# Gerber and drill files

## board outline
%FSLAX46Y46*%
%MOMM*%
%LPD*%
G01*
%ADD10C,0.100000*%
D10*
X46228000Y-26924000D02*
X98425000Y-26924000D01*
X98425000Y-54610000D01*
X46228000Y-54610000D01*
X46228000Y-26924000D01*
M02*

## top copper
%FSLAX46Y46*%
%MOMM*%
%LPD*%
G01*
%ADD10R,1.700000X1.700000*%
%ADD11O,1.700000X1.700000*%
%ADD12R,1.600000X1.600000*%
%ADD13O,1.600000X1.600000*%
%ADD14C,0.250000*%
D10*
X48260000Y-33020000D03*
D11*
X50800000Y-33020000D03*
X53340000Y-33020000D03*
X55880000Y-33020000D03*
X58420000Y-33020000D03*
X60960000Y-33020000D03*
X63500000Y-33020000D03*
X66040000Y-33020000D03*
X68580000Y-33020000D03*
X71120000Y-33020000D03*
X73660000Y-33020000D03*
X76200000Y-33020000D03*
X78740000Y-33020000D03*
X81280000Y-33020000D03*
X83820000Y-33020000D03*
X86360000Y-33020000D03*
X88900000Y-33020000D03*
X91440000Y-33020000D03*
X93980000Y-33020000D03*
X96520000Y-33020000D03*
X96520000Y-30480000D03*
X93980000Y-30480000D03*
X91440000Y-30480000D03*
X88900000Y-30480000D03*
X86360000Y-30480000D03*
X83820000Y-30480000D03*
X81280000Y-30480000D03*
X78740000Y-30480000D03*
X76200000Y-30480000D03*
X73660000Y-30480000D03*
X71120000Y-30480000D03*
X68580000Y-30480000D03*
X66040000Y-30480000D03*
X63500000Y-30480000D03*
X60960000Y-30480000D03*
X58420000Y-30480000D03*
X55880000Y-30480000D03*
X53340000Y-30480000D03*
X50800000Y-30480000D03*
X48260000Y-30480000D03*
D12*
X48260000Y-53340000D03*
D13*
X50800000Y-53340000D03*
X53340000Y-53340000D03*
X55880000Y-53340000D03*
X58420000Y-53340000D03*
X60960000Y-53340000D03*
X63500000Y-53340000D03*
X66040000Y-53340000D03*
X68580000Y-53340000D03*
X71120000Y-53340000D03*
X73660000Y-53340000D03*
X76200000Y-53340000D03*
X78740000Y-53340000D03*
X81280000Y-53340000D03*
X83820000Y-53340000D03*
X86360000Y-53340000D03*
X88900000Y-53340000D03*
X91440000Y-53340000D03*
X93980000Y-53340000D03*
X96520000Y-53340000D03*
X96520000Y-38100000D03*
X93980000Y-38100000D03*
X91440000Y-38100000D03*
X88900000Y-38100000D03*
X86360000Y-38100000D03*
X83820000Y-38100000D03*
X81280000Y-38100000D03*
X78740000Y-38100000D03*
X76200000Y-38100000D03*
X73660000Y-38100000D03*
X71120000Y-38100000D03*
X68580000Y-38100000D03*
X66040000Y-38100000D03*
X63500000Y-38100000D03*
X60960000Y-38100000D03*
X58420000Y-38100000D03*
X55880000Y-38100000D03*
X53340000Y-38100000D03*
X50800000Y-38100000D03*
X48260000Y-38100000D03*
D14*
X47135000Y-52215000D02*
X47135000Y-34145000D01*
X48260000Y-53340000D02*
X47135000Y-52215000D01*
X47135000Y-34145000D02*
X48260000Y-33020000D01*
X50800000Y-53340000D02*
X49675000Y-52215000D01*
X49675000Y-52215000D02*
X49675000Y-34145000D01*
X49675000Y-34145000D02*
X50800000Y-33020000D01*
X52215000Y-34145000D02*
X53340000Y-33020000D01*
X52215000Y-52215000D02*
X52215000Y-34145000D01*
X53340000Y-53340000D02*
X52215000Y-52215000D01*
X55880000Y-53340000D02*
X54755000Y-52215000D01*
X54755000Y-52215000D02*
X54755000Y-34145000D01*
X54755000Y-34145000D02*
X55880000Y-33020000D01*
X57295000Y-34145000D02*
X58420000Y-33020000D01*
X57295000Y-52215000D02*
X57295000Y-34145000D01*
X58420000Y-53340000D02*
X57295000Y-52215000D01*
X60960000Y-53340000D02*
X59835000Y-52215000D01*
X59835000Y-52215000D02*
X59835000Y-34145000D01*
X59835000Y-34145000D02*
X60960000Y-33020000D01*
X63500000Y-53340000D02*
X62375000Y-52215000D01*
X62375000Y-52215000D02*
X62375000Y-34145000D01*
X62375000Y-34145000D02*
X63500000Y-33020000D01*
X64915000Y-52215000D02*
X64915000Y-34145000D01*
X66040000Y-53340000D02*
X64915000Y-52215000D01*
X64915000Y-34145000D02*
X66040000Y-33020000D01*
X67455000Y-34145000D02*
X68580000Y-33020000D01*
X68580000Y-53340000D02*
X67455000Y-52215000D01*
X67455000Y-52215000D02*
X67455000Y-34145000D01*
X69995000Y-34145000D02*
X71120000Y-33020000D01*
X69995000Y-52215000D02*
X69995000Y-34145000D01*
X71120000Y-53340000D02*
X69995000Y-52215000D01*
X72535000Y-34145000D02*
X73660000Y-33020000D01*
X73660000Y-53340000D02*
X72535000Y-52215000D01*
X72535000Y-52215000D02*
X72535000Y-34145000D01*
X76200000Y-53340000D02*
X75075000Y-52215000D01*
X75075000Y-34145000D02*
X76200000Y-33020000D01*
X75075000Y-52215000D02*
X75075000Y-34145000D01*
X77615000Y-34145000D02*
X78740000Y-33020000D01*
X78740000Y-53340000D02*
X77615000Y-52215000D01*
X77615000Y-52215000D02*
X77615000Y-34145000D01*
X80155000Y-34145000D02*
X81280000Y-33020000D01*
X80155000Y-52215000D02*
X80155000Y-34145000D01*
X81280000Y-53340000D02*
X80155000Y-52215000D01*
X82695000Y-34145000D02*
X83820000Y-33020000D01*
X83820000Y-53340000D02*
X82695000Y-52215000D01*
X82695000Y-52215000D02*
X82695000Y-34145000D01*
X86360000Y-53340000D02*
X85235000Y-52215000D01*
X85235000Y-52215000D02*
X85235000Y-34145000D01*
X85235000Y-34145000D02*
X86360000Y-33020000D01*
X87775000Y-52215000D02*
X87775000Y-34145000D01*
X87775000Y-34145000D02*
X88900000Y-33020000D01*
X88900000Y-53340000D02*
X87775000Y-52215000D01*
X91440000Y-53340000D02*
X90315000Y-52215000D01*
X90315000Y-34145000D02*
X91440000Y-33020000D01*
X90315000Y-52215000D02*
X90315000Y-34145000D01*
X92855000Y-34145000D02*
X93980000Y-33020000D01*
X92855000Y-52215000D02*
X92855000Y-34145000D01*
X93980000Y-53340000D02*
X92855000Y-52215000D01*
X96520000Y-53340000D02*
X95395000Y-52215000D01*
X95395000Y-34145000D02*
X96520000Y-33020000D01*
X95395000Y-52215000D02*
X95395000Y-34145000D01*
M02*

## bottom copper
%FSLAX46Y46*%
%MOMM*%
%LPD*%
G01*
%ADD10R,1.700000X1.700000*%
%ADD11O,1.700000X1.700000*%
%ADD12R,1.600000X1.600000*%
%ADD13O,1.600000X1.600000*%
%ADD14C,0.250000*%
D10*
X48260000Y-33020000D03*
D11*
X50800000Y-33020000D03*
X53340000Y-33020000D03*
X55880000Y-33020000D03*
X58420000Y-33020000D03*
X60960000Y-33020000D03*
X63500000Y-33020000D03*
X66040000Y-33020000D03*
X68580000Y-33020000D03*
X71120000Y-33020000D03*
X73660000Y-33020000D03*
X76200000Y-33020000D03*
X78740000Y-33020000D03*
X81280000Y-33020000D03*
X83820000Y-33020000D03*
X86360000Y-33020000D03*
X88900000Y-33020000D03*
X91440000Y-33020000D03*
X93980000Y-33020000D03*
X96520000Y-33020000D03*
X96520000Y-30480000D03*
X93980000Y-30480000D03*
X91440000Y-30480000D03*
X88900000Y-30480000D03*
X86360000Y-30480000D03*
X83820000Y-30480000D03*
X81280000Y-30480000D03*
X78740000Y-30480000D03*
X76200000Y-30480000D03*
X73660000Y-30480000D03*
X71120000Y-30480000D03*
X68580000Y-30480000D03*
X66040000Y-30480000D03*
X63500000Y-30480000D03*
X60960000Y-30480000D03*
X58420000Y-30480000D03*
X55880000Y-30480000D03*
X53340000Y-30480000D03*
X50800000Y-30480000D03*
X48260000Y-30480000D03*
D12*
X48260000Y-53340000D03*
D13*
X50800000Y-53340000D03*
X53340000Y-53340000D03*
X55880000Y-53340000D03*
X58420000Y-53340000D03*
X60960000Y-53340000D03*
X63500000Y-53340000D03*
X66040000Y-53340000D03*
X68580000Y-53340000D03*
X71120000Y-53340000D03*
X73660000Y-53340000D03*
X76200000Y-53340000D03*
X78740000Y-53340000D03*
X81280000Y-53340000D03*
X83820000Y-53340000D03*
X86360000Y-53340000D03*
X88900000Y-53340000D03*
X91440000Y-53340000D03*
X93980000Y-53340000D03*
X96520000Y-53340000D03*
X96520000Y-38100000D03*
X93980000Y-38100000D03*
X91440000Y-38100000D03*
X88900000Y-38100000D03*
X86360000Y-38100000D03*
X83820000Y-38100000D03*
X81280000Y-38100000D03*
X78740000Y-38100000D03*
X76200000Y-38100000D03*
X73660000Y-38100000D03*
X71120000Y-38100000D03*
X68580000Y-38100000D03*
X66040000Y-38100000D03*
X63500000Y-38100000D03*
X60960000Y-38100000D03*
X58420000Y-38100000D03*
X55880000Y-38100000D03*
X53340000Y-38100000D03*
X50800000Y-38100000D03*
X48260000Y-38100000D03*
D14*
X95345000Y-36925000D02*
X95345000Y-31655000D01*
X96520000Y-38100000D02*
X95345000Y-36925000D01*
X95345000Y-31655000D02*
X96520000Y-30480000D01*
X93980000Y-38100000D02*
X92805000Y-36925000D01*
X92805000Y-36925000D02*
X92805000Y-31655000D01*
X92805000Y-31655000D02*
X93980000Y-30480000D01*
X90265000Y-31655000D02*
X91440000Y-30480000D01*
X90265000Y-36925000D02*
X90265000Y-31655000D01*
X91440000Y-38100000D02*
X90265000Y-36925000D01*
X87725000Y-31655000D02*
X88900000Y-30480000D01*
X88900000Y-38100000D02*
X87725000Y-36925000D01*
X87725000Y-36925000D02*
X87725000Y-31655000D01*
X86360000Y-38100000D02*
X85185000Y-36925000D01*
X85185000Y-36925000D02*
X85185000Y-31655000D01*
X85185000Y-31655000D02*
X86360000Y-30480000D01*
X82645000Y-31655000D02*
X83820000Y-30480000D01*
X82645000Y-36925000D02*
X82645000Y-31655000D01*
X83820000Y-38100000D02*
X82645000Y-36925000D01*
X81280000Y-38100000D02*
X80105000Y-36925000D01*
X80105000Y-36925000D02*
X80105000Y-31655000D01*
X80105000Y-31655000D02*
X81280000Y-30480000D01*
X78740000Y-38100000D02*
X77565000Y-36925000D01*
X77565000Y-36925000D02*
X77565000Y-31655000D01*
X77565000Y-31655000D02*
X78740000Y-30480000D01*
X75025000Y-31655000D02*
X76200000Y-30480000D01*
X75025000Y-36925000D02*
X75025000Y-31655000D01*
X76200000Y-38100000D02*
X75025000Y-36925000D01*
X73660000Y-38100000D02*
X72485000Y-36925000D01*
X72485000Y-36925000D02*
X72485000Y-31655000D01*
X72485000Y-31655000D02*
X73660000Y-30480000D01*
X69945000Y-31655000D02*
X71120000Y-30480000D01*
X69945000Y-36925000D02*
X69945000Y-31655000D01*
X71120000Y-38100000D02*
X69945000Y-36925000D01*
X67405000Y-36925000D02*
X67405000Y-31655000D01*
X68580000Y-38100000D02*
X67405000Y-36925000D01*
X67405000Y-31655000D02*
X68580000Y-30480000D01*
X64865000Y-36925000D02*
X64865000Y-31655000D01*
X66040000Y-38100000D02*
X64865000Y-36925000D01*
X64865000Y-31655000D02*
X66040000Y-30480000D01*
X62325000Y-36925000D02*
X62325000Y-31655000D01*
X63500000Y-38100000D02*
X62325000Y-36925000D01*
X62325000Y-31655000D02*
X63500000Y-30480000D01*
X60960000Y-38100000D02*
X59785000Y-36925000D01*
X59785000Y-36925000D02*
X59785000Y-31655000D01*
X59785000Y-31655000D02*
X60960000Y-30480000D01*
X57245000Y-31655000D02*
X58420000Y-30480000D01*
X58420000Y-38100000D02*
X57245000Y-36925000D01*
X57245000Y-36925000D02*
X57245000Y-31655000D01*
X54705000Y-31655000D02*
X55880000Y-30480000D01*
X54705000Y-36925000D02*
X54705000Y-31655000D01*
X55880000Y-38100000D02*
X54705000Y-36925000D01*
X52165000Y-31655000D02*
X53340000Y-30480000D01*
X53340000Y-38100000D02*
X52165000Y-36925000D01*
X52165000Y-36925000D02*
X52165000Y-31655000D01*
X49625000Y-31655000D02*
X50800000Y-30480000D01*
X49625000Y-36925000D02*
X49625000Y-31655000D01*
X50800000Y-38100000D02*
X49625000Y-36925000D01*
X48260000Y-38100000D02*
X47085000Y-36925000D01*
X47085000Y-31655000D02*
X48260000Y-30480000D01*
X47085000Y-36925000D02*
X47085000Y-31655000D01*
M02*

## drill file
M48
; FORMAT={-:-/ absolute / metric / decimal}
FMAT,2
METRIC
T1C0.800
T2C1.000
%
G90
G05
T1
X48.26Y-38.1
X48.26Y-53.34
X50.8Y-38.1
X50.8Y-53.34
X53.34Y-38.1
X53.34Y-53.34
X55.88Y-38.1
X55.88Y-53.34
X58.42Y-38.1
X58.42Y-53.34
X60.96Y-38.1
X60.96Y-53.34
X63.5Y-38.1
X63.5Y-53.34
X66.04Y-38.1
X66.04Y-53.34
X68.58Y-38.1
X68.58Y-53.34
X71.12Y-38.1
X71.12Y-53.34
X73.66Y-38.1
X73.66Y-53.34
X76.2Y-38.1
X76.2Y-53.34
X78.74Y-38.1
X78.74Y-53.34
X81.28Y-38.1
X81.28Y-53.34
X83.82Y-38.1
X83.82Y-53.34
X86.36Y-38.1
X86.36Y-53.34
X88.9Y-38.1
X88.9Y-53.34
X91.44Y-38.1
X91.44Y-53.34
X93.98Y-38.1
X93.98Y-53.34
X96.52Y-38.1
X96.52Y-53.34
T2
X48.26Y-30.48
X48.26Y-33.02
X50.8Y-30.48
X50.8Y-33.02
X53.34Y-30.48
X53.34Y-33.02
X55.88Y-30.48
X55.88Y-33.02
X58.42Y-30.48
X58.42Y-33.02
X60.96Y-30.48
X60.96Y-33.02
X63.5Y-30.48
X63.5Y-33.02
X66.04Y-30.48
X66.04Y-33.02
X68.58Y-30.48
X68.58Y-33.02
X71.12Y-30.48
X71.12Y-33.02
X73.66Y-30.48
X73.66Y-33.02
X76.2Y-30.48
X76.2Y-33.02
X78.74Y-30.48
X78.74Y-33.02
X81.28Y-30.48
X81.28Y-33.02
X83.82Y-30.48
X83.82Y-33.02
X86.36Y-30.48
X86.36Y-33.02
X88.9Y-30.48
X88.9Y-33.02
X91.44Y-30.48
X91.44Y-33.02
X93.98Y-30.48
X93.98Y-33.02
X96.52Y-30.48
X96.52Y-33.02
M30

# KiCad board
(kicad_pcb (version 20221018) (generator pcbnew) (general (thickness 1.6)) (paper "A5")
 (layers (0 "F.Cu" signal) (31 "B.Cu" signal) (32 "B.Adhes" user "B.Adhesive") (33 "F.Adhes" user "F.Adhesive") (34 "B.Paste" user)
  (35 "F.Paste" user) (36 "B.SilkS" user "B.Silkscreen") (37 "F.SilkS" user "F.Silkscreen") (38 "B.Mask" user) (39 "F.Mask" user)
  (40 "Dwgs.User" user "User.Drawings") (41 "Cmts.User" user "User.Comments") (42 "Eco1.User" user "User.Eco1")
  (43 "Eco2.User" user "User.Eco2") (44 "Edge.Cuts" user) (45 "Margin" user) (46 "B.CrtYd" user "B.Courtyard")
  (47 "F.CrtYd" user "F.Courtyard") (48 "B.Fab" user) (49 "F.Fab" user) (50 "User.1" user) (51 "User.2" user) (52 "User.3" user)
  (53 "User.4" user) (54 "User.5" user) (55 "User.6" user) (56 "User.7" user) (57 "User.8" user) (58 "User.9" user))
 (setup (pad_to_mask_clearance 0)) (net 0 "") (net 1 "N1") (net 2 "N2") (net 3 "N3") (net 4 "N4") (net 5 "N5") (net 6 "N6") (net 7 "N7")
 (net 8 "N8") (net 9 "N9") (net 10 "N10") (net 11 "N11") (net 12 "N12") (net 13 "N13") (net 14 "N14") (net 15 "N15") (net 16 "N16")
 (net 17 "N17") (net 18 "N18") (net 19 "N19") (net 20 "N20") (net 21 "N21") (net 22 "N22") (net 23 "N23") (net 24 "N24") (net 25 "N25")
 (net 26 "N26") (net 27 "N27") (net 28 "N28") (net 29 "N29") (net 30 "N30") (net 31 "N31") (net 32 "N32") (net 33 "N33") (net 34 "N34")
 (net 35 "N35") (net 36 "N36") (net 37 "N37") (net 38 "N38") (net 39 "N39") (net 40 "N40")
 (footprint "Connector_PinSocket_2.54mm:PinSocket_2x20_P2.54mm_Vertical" (layer "F.Cu") (at 48.26 33.02 90)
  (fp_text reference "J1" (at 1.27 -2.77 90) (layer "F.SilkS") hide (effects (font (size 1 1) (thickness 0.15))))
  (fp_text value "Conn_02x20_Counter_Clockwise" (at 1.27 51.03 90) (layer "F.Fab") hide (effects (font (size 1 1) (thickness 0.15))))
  (pad "1" thru_hole rect (at 0 0 90) (size 1.7 1.7) (drill 1) (layers "*.Cu" "*.Mask") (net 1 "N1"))
  (pad "2" thru_hole oval (at 0 2.54 90) (size 1.7 1.7) (drill 1) (layers "*.Cu" "*.Mask") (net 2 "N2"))
  (pad "3" thru_hole oval (at 0 5.08 90) (size 1.7 1.7) (drill 1) (layers "*.Cu" "*.Mask") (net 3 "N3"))
  (pad "4" thru_hole oval (at 0 7.62 90) (size 1.7 1.7) (drill 1) (layers "*.Cu" "*.Mask") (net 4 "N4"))
  (pad "5" thru_hole oval (at 0 10.16 90) (size 1.7 1.7) (drill 1) (layers "*.Cu" "*.Mask") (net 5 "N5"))
  (pad "6" thru_hole oval (at 0 12.7 90) (size 1.7 1.7) (drill 1) (layers "*.Cu" "*.Mask") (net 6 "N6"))
  (pad "7" thru_hole oval (at 0 15.24 90) (size 1.7 1.7) (drill 1) (layers "*.Cu" "*.Mask") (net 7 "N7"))
  (pad "8" thru_hole oval (at 0 17.78 90) (size 1.7 1.7) (drill 1) (layers "*.Cu" "*.Mask") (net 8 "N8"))
  (pad "9" thru_hole oval (at 0 20.32 90) (size 1.7 1.7) (drill 1) (layers "*.Cu" "*.Mask") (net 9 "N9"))
  (pad "10" thru_hole oval (at 0 22.86 90) (size 1.7 1.7) (drill 1) (layers "*.Cu" "*.Mask") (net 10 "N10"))
  (pad "11" thru_hole oval (at 0 25.4 90) (size 1.7 1.7) (drill 1) (layers "*.Cu" "*.Mask") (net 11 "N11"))
  (pad "12" thru_hole oval (at 0 27.94 90) (size 1.7 1.7) (drill 1) (layers "*.Cu" "*.Mask") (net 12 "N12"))
  (pad "13" thru_hole oval (at 0 30.48 90) (size 1.7 1.7) (drill 1) (layers "*.Cu" "*.Mask") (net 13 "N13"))
  (pad "14" thru_hole oval (at 0 33.02 90) (size 1.7 1.7) (drill 1) (layers "*.Cu" "*.Mask") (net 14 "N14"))
  (pad "15" thru_hole oval (at 0 35.56 90) (size 1.7 1.7) (drill 1) (layers "*.Cu" "*.Mask") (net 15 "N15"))
  (pad "16" thru_hole oval (at 0 38.1 90) (size 1.7 1.7) (drill 1) (layers "*.Cu" "*.Mask") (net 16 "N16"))
  (pad "17" thru_hole oval (at 0 40.64 90) (size 1.7 1.7) (drill 1) (layers "*.Cu" "*.Mask") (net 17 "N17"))
  (pad "18" thru_hole oval (at 0 43.18 90) (size 1.7 1.7) (drill 1) (layers "*.Cu" "*.Mask") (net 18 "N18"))
  (pad "19" thru_hole oval (at 0 45.72 90) (size 1.7 1.7) (drill 1) (layers "*.Cu" "*.Mask") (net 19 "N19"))
  (pad "20" thru_hole oval (at 0 48.26 90) (size 1.7 1.7) (drill 1) (layers "*.Cu" "*.Mask") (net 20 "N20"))
  (pad "21" thru_hole oval (at 2.54 48.26 90) (size 1.7 1.7) (drill 1) (layers "*.Cu" "*.Mask") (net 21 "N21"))
  (pad "22" thru_hole oval (at 2.54 45.72 90) (size 1.7 1.7) (drill 1) (layers "*.Cu" "*.Mask") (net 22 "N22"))
  (pad "23" thru_hole oval (at 2.54 43.18 90) (size 1.7 1.7) (drill 1) (layers "*.Cu" "*.Mask") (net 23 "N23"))
  (pad "24" thru_hole oval (at 2.54 40.64 90) (size 1.7 1.7) (drill 1) (layers "*.Cu" "*.Mask") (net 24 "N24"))
  (pad "25" thru_hole oval (at 2.54 38.1 90) (size 1.7 1.7) (drill 1) (layers "*.Cu" "*.Mask") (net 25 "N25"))
  (pad "26" thru_hole oval (at 2.54 35.56 90) (size 1.7 1.7) (drill 1) (layers "*.Cu" "*.Mask") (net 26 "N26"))
  (pad "27" thru_hole oval (at 2.54 33.02 90) (size 1.7 1.7) (drill 1) (layers "*.Cu" "*.Mask") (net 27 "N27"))
  (pad "28" thru_hole oval (at 2.54 30.48 90) (size 1.7 1.7) (drill 1) (layers "*.Cu" "*.Mask") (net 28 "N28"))
  (pad "29" thru_hole oval (at 2.54 27.94 90) (size 1.7 1.7) (drill 1) (layers "*.Cu" "*.Mask") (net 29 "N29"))
  (pad "30" thru_hole oval (at 2.54 25.4 90) (size 1.7 1.7) (drill 1) (layers "*.Cu" "*.Mask") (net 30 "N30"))
  (pad "31" thru_hole oval (at 2.54 22.86 90) (size 1.7 1.7) (drill 1) (layers "*.Cu" "*.Mask") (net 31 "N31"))
  (pad "32" thru_hole oval (at 2.54 20.32 90) (size 1.7 1.7) (drill 1) (layers "*.Cu" "*.Mask") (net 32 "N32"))
  (pad "33" thru_hole oval (at 2.54 17.78 90) (size 1.7 1.7) (drill 1) (layers "*.Cu" "*.Mask") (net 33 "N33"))
  (pad "34" thru_hole oval (at 2.54 15.24 90) (size 1.7 1.7) (drill 1) (layers "*.Cu" "*.Mask") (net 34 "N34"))
  (pad "35" thru_hole oval (at 2.54 12.7 90) (size 1.7 1.7) (drill 1) (layers "*.Cu" "*.Mask") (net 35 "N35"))
  (pad "36" thru_hole oval (at 2.54 10.16 90) (size 1.7 1.7) (drill 1) (layers "*.Cu" "*.Mask") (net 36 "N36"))
  (pad "37" thru_hole oval (at 2.54 7.62 90) (size 1.7 1.7) (drill 1) (layers "*.Cu" "*.Mask") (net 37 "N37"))
  (pad "38" thru_hole oval (at 2.54 5.08 90) (size 1.7 1.7) (drill 1) (layers "*.Cu" "*.Mask") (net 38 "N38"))
  (pad "39" thru_hole oval (at 2.54 2.54 90) (size 1.7 1.7) (drill 1) (layers "*.Cu" "*.Mask") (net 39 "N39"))
  (pad "40" thru_hole oval (at 2.54 0 90) (size 1.7 1.7) (drill 1) (layers "*.Cu" "*.Mask") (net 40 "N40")))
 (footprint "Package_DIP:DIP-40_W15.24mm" (layer "F.Cu") (at 48.26 53.34 90)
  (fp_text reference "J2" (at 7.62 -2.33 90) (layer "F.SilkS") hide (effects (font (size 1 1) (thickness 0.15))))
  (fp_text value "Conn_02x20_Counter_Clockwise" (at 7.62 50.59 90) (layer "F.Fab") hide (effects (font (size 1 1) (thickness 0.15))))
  (pad "1" thru_hole rect (at 0 0 90) (size 1.6 1.6) (drill 0.8) (layers "*.Cu" "*.Mask") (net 1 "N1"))
  (pad "2" thru_hole oval (at 0 2.54 90) (size 1.6 1.6) (drill 0.8) (layers "*.Cu" "*.Mask") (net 2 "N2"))
  (pad "3" thru_hole oval (at 0 5.08 90) (size 1.6 1.6) (drill 0.8) (layers "*.Cu" "*.Mask") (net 3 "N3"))
  (pad "4" thru_hole oval (at 0 7.62 90) (size 1.6 1.6) (drill 0.8) (layers "*.Cu" "*.Mask") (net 4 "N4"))
  (pad "5" thru_hole oval (at 0 10.16 90) (size 1.6 1.6) (drill 0.8) (layers "*.Cu" "*.Mask") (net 5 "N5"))
  (pad "6" thru_hole oval (at 0 12.7 90) (size 1.6 1.6) (drill 0.8) (layers "*.Cu" "*.Mask") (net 6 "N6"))
  (pad "7" thru_hole oval (at 0 15.24 90) (size 1.6 1.6) (drill 0.8) (layers "*.Cu" "*.Mask") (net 7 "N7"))
  (pad "8" thru_hole oval (at 0 17.78 90) (size 1.6 1.6) (drill 0.8) (layers "*.Cu" "*.Mask") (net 8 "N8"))
  (pad "9" thru_hole oval (at 0 20.32 90) (size 1.6 1.6) (drill 0.8) (layers "*.Cu" "*.Mask") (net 9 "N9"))
  (pad "10" thru_hole oval (at 0 22.86 90) (size 1.6 1.6) (drill 0.8) (layers "*.Cu" "*.Mask") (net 10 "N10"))
  (pad "11" thru_hole oval (at 0 25.4 90) (size 1.6 1.6) (drill 0.8) (layers "*.Cu" "*.Mask") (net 11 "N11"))
  (pad "12" thru_hole oval (at 0 27.94 90) (size 1.6 1.6) (drill 0.8) (layers "*.Cu" "*.Mask") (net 12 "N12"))
  (pad "13" thru_hole oval (at 0 30.48 90) (size 1.6 1.6) (drill 0.8) (layers "*.Cu" "*.Mask") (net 13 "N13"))
  (pad "14" thru_hole oval (at 0 33.02 90) (size 1.6 1.6) (drill 0.8) (layers "*.Cu" "*.Mask") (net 14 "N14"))
  (pad "15" thru_hole oval (at 0 35.56 90) (size 1.6 1.6) (drill 0.8) (layers "*.Cu" "*.Mask") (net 15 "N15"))
  (pad "16" thru_hole oval (at 0 38.1 90) (size 1.6 1.6) (drill 0.8) (layers "*.Cu" "*.Mask") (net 16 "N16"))
  (pad "17" thru_hole oval (at 0 40.64 90) (size 1.6 1.6) (drill 0.8) (layers "*.Cu" "*.Mask") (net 17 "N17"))
  (pad "18" thru_hole oval (at 0 43.18 90) (size 1.6 1.6) (drill 0.8) (layers "*.Cu" "*.Mask") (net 18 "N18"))
  (pad "19" thru_hole oval (at 0 45.72 90) (size 1.6 1.6) (drill 0.8) (layers "*.Cu" "*.Mask") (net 19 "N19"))
  (pad "20" thru_hole oval (at 0 48.26 90) (size 1.6 1.6) (drill 0.8) (layers "*.Cu" "*.Mask") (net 20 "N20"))
  (pad "21" thru_hole oval (at 15.24 48.26 90) (size 1.6 1.6) (drill 0.8) (layers "*.Cu" "*.Mask") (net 21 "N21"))
  (pad "22" thru_hole oval (at 15.24 45.72 90) (size 1.6 1.6) (drill 0.8) (layers "*.Cu" "*.Mask") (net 22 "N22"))
  (pad "23" thru_hole oval (at 15.24 43.18 90) (size 1.6 1.6) (drill 0.8) (layers "*.Cu" "*.Mask") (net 23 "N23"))
  (pad "24" thru_hole oval (at 15.24 40.64 90) (size 1.6 1.6) (drill 0.8) (layers "*.Cu" "*.Mask") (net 24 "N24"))
  (pad "25" thru_hole oval (at 15.24 38.1 90) (size 1.6 1.6) (drill 0.8) (layers "*.Cu" "*.Mask") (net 25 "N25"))
  (pad "26" thru_hole oval (at 15.24 35.56 90) (size 1.6 1.6) (drill 0.8) (layers "*.Cu" "*.Mask") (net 26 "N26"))
  (pad "27" thru_hole oval (at 15.24 33.02 90) (size 1.6 1.6) (drill 0.8) (layers "*.Cu" "*.Mask") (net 27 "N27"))
  (pad "28" thru_hole oval (at 15.24 30.48 90) (size 1.6 1.6) (drill 0.8) (layers "*.Cu" "*.Mask") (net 28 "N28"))
  (pad "29" thru_hole oval (at 15.24 27.94 90) (size 1.6 1.6) (drill 0.8) (layers "*.Cu" "*.Mask") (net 29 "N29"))
  (pad "30" thru_hole oval (at 15.24 25.4 90) (size 1.6 1.6) (drill 0.8) (layers "*.Cu" "*.Mask") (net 30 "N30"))
  (pad "31" thru_hole oval (at 15.24 22.86 90) (size 1.6 1.6) (drill 0.8) (layers "*.Cu" "*.Mask") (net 31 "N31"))
  (pad "32" thru_hole oval (at 15.24 20.32 90) (size 1.6 1.6) (drill 0.8) (layers "*.Cu" "*.Mask") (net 32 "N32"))
  (pad "33" thru_hole oval (at 15.24 17.78 90) (size 1.6 1.6) (drill 0.8) (layers "*.Cu" "*.Mask") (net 33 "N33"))
  (pad "34" thru_hole oval (at 15.24 15.24 90) (size 1.6 1.6) (drill 0.8) (layers "*.Cu" "*.Mask") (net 34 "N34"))
  (pad "35" thru_hole oval (at 15.24 12.7 90) (size 1.6 1.6) (drill 0.8) (layers "*.Cu" "*.Mask") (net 35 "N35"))
  (pad "36" thru_hole oval (at 15.24 10.16 90) (size 1.6 1.6) (drill 0.8) (layers "*.Cu" "*.Mask") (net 36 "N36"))
  (pad "37" thru_hole oval (at 15.24 7.62 90) (size 1.6 1.6) (drill 0.8) (layers "*.Cu" "*.Mask") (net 37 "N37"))
  (pad "38" thru_hole oval (at 15.24 5.08 90) (size 1.6 1.6) (drill 0.8) (layers "*.Cu" "*.Mask") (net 38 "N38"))
  (pad "39" thru_hole oval (at 15.24 2.54 90) (size 1.6 1.6) (drill 0.8) (layers "*.Cu" "*.Mask") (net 39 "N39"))
  (pad "40" thru_hole oval (at 15.24 0 90) (size 1.6 1.6) (drill 0.8) (layers "*.Cu" "*.Mask") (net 40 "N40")))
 (gr_rect (start 46.228 26.924) (end 98.425 54.61) (stroke (width 0.1) (type default)) (fill none) (layer "Edge.Cuts"))
 (segment (start 47.135 52.215) (end 47.135 34.145) (width 0.25) (layer "F.Cu") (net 1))
 (segment (start 48.26 53.34) (end 47.135 52.215) (width 0.25) (layer "F.Cu") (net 1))
 (segment (start 47.135 34.145) (end 48.26 33.02) (width 0.25) (layer "F.Cu") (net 1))
 (segment (start 50.8 53.34) (end 49.675 52.215) (width 0.25) (layer "F.Cu") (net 2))
 (segment (start 49.675 52.215) (end 49.675 34.145) (width 0.25) (layer "F.Cu") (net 2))
 (segment (start 49.675 34.145) (end 50.8 33.02) (width 0.25) (layer "F.Cu") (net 2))
 (segment (start 52.215 34.145) (end 53.34 33.02) (width 0.25) (layer "F.Cu") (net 3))
 (segment (start 52.215 52.215) (end 52.215 34.145) (width 0.25) (layer "F.Cu") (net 3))
 (segment (start 53.34 53.34) (end 52.215 52.215) (width 0.25) (layer "F.Cu") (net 3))
 (segment (start 55.88 53.34) (end 54.755 52.215) (width 0.25) (layer "F.Cu") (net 4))
 (segment (start 54.755 52.215) (end 54.755 34.145) (width 0.25) (layer "F.Cu") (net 4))
 (segment (start 54.755 34.145) (end 55.88 33.02) (width 0.25) (layer "F.Cu") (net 4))
 (segment (start 57.295 34.145) (end 58.42 33.02) (width 0.25) (layer "F.Cu") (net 5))
 (segment (start 57.295 52.215) (end 57.295 34.145) (width 0.25) (layer "F.Cu") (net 5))
 (segment (start 58.42 53.34) (end 57.295 52.215) (width 0.25) (layer "F.Cu") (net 5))
 (segment (start 60.96 53.34) (end 59.835 52.215) (width 0.25) (layer "F.Cu") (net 6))
 (segment (start 59.835 52.215) (end 59.835 34.145) (width 0.25) (layer "F.Cu") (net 6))
 (segment (start 59.835 34.145) (end 60.96 33.02) (width 0.25) (layer "F.Cu") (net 6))
 (segment (start 63.5 53.34) (end 62.375 52.215) (width 0.25) (layer "F.Cu") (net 7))
 (segment (start 62.375 52.215) (end 62.375 34.145) (width 0.25) (layer "F.Cu") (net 7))
 (segment (start 62.375 34.145) (end 63.5 33.02) (width 0.25) (layer "F.Cu") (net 7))
 (segment (start 64.915 52.215) (end 64.915 34.145) (width 0.25) (layer "F.Cu") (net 8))
 (segment (start 66.04 53.34) (end 64.915 52.215) (width 0.25) (layer "F.Cu") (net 8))
 (segment (start 64.915 34.145) (end 66.04 33.02) (width 0.25) (layer "F.Cu") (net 8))
 (segment (start 67.455 34.145) (end 68.58 33.02) (width 0.25) (layer "F.Cu") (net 9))
 (segment (start 68.58 53.34) (end 67.455 52.215) (width 0.25) (layer "F.Cu") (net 9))
 (segment (start 67.455 52.215) (end 67.455 34.145) (width 0.25) (layer "F.Cu") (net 9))
 (segment (start 69.995 34.145) (end 71.12 33.02) (width 0.25) (layer "F.Cu") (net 10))
 (segment (start 69.995 52.215) (end 69.995 34.145) (width 0.25) (layer "F.Cu") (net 10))
 (segment (start 71.12 53.34) (end 69.995 52.215) (width 0.25) (layer "F.Cu") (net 10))
 (segment (start 72.535 34.145) (end 73.66 33.02) (width 0.25) (layer "F.Cu") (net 11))
 (segment (start 73.66 53.34) (end 72.535 52.215) (width 0.25) (layer "F.Cu") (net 11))
 (segment (start 72.535 52.215) (end 72.535 34.145) (width 0.25) (layer "F.Cu") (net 11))
 (segment (start 76.2 53.34) (end 75.075 52.215) (width 0.25) (layer "F.Cu") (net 12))
 (segment (start 75.075 34.145) (end 76.2 33.02) (width 0.25) (layer "F.Cu") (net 12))
 (segment (start 75.075 52.215) (end 75.075 34.145) (width 0.25) (layer "F.Cu") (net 12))
 (segment (start 77.615 34.145) (end 78.74 33.02) (width 0.25) (layer "F.Cu") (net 13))
 (segment (start 78.74 53.34) (end 77.615 52.215) (width 0.25) (layer "F.Cu") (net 13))
 (segment (start 77.615 52.215) (end 77.615 34.145) (width 0.25) (layer "F.Cu") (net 13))
 (segment (start 80.155 34.145) (end 81.28 33.02) (width 0.25) (layer "F.Cu") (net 14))
 (segment (start 80.155 52.215) (end 80.155 34.145) (width 0.25) (layer "F.Cu") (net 14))
 (segment (start 81.28 53.34) (end 80.155 52.215) (width 0.25) (layer "F.Cu") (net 14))
 (segment (start 82.695 34.145) (end 83.82 33.02) (width 0.25) (layer "F.Cu") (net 15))
 (segment (start 83.82 53.34) (end 82.695 52.215) (width 0.25) (layer "F.Cu") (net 15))
 (segment (start 82.695 52.215) (end 82.695 34.145) (width 0.25) (layer "F.Cu") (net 15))
 (segment (start 86.36 53.34) (end 85.235 52.215) (width 0.25) (layer "F.Cu") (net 16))
 (segment (start 85.235 52.215) (end 85.235 34.145) (width 0.25) (layer "F.Cu") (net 16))
 (segment (start 85.235 34.145) (end 86.36 33.02) (width 0.25) (layer "F.Cu") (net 16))
 (segment (start 87.775 52.215) (end 87.775 34.145) (width 0.25) (layer "F.Cu") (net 17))
 (segment (start 87.775 34.145) (end 88.9 33.02) (width 0.25) (layer "F.Cu") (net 17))
 (segment (start 88.9 53.34) (end 87.775 52.215) (width 0.25) (layer "F.Cu") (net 17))
 (segment (start 91.44 53.34) (end 90.315 52.215) (width 0.25) (layer "F.Cu") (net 18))
 (segment (start 90.315 34.145) (end 91.44 33.02) (width 0.25) (layer "F.Cu") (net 18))
 (segment (start 90.315 52.215) (end 90.315 34.145) (width 0.25) (layer "F.Cu") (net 18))
 (segment (start 92.855 34.145) (end 93.98 33.02) (width 0.25) (layer "F.Cu") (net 19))
 (segment (start 92.855 52.215) (end 92.855 34.145) (width 0.25) (layer "F.Cu") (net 19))
 (segment (start 93.98 53.34) (end 92.855 52.215) (width 0.25) (layer "F.Cu") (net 19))
 (segment (start 96.52 53.34) (end 95.395 52.215) (width 0.25) (layer "F.Cu") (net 20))
 (segment (start 95.395 34.145) (end 96.52 33.02) (width 0.25) (layer "F.Cu") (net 20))
 (segment (start 95.395 52.215) (end 95.395 34.145) (width 0.25) (layer "F.Cu") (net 20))
 (segment (start 95.345 36.925) (end 95.345 31.655) (width 0.25) (layer "B.Cu") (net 21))
 (segment (start 96.52 38.1) (end 95.345 36.925) (width 0.25) (layer "B.Cu") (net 21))
 (segment (start 95.345 31.655) (end 96.52 30.48) (width 0.25) (layer "B.Cu") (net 21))
 (segment (start 93.98 38.1) (end 92.805 36.925) (width 0.25) (layer "B.Cu") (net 22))
 (segment (start 92.805 36.925) (end 92.805 31.655) (width 0.25) (layer "B.Cu") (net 22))
 (segment (start 92.805 31.655) (end 93.98 30.48) (width 0.25) (layer "B.Cu") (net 22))
 (segment (start 90.265 31.655) (end 91.44 30.48) (width 0.25) (layer "B.Cu") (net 23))
 (segment (start 90.265 36.925) (end 90.265 31.655) (width 0.25) (layer "B.Cu") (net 23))
 (segment (start 91.44 38.1) (end 90.265 36.925) (width 0.25) (layer "B.Cu") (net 23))
 (segment (start 87.725 31.655) (end 88.9 30.48) (width 0.25) (layer "B.Cu") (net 24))
 (segment (start 88.9 38.1) (end 87.725 36.925) (width 0.25) (layer "B.Cu") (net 24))
 (segment (start 87.725 36.925) (end 87.725 31.655) (width 0.25) (layer "B.Cu") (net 24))
 (segment (start 86.36 38.1) (end 85.185 36.925) (width 0.25) (layer "B.Cu") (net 25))
 (segment (start 85.185 36.925) (end 85.185 31.655) (width 0.25) (layer "B.Cu") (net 25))
 (segment (start 85.185 31.655) (end 86.36 30.48) (width 0.25) (layer "B.Cu") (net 25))
 (segment (start 82.645 31.655) (end 83.82 30.48) (width 0.25) (layer "B.Cu") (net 26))
 (segment (start 82.645 36.925) (end 82.645 31.655) (width 0.25) (layer "B.Cu") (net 26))
 (segment (start 83.82 38.1) (end 82.645 36.925) (width 0.25) (layer "B.Cu") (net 26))
 (segment (start 81.28 38.1) (end 80.105 36.925) (width 0.25) (layer "B.Cu") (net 27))
 (segment (start 80.105 36.925) (end 80.105 31.655) (width 0.25) (layer "B.Cu") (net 27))
 (segment (start 80.105 31.655) (end 81.28 30.48) (width 0.25) (layer "B.Cu") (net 27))
 (segment (start 78.74 38.1) (end 77.565 36.925) (width 0.25) (layer "B.Cu") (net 28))
 (segment (start 77.565 36.925) (end 77.565 31.655) (width 0.25) (layer "B.Cu") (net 28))
 (segment (start 77.565 31.655) (end 78.74 30.48) (width 0.25) (layer "B.Cu") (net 28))
 (segment (start 75.025 31.655) (end 76.2 30.48) (width 0.25) (layer "B.Cu") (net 29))
 (segment (start 75.025 36.925) (end 75.025 31.655) (width 0.25) (layer "B.Cu") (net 29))
 (segment (start 76.2 38.1) (end 75.025 36.925) (width 0.25) (layer "B.Cu") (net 29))
 (segment (start 73.66 38.1) (end 72.485 36.925) (width 0.25) (layer "B.Cu") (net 30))
 (segment (start 72.485 36.925) (end 72.485 31.655) (width 0.25) (layer "B.Cu") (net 30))
 (segment (start 72.485 31.655) (end 73.66 30.48) (width 0.25) (layer "B.Cu") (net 30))
 (segment (start 69.945 31.655) (end 71.12 30.48) (width 0.25) (layer "B.Cu") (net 31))
 (segment (start 69.945 36.925) (end 69.945 31.655) (width 0.25) (layer "B.Cu") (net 31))
 (segment (start 71.12 38.1) (end 69.945 36.925) (width 0.25) (layer "B.Cu") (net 31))
 (segment (start 67.405 36.925) (end 67.405 31.655) (width 0.25) (layer "B.Cu") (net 32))
 (segment (start 68.58 38.1) (end 67.405 36.925) (width 0.25) (layer "B.Cu") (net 32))
 (segment (start 67.405 31.655) (end 68.58 30.48) (width 0.25) (layer "B.Cu") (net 32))
 (segment (start 64.865 36.925) (end 64.865 31.655) (width 0.25) (layer "B.Cu") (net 33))
 (segment (start 66.04 38.1) (end 64.865 36.925) (width 0.25) (layer "B.Cu") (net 33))
 (segment (start 64.865 31.655) (end 66.04 30.48) (width 0.25) (layer "B.Cu") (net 33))
 (segment (start 62.325 36.925) (end 62.325 31.655) (width 0.25) (layer "B.Cu") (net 34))
 (segment (start 63.5 38.1) (end 62.325 36.925) (width 0.25) (layer "B.Cu") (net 34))
 (segment (start 62.325 31.655) (end 63.5 30.48) (width 0.25) (layer "B.Cu") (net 34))
 (segment (start 60.96 38.1) (end 59.785 36.925) (width 0.25) (layer "B.Cu") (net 35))
 (segment (start 59.785 36.925) (end 59.785 31.655) (width 0.25) (layer "B.Cu") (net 35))
 (segment (start 59.785 31.655) (end 60.96 30.48) (width 0.25) (layer "B.Cu") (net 35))
 (segment (start 57.245 31.655) (end 58.42 30.48) (width 0.25) (layer "B.Cu") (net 36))
 (segment (start 58.42 38.1) (end 57.245 36.925) (width 0.25) (layer "B.Cu") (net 36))
 (segment (start 57.245 36.925) (end 57.245 31.655) (width 0.25) (layer "B.Cu") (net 36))
 (segment (start 54.705 31.655) (end 55.88 30.48) (width 0.25) (layer "B.Cu") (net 37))
 (segment (start 54.705 36.925) (end 54.705 31.655) (width 0.25) (layer "B.Cu") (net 37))
 (segment (start 55.88 38.1) (end 54.705 36.925) (width 0.25) (layer "B.Cu") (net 37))
 (segment (start 52.165 31.655) (end 53.34 30.48) (width 0.25) (layer "B.Cu") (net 38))
 (segment (start 53.34 38.1) (end 52.165 36.925) (width 0.25) (layer "B.Cu") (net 38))
 (segment (start 52.165 36.925) (end 52.165 31.655) (width 0.25) (layer "B.Cu") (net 38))
 (segment (start 49.625 31.655) (end 50.8 30.48) (width 0.25) (layer "B.Cu") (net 39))
 (segment (start 49.625 36.925) (end 49.625 31.655) (width 0.25) (layer "B.Cu") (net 39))
 (segment (start 50.8 38.1) (end 49.625 36.925) (width 0.25) (layer "B.Cu") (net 39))
 (segment (start 48.26 38.1) (end 47.085 36.925) (width 0.25) (layer "B.Cu") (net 40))
 (segment (start 47.085 31.655) (end 48.26 30.48) (width 0.25) (layer "B.Cu") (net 40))
 (segment (start 47.085 36.925) (end 47.085 31.655) (width 0.25) (layer "B.Cu") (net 40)))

